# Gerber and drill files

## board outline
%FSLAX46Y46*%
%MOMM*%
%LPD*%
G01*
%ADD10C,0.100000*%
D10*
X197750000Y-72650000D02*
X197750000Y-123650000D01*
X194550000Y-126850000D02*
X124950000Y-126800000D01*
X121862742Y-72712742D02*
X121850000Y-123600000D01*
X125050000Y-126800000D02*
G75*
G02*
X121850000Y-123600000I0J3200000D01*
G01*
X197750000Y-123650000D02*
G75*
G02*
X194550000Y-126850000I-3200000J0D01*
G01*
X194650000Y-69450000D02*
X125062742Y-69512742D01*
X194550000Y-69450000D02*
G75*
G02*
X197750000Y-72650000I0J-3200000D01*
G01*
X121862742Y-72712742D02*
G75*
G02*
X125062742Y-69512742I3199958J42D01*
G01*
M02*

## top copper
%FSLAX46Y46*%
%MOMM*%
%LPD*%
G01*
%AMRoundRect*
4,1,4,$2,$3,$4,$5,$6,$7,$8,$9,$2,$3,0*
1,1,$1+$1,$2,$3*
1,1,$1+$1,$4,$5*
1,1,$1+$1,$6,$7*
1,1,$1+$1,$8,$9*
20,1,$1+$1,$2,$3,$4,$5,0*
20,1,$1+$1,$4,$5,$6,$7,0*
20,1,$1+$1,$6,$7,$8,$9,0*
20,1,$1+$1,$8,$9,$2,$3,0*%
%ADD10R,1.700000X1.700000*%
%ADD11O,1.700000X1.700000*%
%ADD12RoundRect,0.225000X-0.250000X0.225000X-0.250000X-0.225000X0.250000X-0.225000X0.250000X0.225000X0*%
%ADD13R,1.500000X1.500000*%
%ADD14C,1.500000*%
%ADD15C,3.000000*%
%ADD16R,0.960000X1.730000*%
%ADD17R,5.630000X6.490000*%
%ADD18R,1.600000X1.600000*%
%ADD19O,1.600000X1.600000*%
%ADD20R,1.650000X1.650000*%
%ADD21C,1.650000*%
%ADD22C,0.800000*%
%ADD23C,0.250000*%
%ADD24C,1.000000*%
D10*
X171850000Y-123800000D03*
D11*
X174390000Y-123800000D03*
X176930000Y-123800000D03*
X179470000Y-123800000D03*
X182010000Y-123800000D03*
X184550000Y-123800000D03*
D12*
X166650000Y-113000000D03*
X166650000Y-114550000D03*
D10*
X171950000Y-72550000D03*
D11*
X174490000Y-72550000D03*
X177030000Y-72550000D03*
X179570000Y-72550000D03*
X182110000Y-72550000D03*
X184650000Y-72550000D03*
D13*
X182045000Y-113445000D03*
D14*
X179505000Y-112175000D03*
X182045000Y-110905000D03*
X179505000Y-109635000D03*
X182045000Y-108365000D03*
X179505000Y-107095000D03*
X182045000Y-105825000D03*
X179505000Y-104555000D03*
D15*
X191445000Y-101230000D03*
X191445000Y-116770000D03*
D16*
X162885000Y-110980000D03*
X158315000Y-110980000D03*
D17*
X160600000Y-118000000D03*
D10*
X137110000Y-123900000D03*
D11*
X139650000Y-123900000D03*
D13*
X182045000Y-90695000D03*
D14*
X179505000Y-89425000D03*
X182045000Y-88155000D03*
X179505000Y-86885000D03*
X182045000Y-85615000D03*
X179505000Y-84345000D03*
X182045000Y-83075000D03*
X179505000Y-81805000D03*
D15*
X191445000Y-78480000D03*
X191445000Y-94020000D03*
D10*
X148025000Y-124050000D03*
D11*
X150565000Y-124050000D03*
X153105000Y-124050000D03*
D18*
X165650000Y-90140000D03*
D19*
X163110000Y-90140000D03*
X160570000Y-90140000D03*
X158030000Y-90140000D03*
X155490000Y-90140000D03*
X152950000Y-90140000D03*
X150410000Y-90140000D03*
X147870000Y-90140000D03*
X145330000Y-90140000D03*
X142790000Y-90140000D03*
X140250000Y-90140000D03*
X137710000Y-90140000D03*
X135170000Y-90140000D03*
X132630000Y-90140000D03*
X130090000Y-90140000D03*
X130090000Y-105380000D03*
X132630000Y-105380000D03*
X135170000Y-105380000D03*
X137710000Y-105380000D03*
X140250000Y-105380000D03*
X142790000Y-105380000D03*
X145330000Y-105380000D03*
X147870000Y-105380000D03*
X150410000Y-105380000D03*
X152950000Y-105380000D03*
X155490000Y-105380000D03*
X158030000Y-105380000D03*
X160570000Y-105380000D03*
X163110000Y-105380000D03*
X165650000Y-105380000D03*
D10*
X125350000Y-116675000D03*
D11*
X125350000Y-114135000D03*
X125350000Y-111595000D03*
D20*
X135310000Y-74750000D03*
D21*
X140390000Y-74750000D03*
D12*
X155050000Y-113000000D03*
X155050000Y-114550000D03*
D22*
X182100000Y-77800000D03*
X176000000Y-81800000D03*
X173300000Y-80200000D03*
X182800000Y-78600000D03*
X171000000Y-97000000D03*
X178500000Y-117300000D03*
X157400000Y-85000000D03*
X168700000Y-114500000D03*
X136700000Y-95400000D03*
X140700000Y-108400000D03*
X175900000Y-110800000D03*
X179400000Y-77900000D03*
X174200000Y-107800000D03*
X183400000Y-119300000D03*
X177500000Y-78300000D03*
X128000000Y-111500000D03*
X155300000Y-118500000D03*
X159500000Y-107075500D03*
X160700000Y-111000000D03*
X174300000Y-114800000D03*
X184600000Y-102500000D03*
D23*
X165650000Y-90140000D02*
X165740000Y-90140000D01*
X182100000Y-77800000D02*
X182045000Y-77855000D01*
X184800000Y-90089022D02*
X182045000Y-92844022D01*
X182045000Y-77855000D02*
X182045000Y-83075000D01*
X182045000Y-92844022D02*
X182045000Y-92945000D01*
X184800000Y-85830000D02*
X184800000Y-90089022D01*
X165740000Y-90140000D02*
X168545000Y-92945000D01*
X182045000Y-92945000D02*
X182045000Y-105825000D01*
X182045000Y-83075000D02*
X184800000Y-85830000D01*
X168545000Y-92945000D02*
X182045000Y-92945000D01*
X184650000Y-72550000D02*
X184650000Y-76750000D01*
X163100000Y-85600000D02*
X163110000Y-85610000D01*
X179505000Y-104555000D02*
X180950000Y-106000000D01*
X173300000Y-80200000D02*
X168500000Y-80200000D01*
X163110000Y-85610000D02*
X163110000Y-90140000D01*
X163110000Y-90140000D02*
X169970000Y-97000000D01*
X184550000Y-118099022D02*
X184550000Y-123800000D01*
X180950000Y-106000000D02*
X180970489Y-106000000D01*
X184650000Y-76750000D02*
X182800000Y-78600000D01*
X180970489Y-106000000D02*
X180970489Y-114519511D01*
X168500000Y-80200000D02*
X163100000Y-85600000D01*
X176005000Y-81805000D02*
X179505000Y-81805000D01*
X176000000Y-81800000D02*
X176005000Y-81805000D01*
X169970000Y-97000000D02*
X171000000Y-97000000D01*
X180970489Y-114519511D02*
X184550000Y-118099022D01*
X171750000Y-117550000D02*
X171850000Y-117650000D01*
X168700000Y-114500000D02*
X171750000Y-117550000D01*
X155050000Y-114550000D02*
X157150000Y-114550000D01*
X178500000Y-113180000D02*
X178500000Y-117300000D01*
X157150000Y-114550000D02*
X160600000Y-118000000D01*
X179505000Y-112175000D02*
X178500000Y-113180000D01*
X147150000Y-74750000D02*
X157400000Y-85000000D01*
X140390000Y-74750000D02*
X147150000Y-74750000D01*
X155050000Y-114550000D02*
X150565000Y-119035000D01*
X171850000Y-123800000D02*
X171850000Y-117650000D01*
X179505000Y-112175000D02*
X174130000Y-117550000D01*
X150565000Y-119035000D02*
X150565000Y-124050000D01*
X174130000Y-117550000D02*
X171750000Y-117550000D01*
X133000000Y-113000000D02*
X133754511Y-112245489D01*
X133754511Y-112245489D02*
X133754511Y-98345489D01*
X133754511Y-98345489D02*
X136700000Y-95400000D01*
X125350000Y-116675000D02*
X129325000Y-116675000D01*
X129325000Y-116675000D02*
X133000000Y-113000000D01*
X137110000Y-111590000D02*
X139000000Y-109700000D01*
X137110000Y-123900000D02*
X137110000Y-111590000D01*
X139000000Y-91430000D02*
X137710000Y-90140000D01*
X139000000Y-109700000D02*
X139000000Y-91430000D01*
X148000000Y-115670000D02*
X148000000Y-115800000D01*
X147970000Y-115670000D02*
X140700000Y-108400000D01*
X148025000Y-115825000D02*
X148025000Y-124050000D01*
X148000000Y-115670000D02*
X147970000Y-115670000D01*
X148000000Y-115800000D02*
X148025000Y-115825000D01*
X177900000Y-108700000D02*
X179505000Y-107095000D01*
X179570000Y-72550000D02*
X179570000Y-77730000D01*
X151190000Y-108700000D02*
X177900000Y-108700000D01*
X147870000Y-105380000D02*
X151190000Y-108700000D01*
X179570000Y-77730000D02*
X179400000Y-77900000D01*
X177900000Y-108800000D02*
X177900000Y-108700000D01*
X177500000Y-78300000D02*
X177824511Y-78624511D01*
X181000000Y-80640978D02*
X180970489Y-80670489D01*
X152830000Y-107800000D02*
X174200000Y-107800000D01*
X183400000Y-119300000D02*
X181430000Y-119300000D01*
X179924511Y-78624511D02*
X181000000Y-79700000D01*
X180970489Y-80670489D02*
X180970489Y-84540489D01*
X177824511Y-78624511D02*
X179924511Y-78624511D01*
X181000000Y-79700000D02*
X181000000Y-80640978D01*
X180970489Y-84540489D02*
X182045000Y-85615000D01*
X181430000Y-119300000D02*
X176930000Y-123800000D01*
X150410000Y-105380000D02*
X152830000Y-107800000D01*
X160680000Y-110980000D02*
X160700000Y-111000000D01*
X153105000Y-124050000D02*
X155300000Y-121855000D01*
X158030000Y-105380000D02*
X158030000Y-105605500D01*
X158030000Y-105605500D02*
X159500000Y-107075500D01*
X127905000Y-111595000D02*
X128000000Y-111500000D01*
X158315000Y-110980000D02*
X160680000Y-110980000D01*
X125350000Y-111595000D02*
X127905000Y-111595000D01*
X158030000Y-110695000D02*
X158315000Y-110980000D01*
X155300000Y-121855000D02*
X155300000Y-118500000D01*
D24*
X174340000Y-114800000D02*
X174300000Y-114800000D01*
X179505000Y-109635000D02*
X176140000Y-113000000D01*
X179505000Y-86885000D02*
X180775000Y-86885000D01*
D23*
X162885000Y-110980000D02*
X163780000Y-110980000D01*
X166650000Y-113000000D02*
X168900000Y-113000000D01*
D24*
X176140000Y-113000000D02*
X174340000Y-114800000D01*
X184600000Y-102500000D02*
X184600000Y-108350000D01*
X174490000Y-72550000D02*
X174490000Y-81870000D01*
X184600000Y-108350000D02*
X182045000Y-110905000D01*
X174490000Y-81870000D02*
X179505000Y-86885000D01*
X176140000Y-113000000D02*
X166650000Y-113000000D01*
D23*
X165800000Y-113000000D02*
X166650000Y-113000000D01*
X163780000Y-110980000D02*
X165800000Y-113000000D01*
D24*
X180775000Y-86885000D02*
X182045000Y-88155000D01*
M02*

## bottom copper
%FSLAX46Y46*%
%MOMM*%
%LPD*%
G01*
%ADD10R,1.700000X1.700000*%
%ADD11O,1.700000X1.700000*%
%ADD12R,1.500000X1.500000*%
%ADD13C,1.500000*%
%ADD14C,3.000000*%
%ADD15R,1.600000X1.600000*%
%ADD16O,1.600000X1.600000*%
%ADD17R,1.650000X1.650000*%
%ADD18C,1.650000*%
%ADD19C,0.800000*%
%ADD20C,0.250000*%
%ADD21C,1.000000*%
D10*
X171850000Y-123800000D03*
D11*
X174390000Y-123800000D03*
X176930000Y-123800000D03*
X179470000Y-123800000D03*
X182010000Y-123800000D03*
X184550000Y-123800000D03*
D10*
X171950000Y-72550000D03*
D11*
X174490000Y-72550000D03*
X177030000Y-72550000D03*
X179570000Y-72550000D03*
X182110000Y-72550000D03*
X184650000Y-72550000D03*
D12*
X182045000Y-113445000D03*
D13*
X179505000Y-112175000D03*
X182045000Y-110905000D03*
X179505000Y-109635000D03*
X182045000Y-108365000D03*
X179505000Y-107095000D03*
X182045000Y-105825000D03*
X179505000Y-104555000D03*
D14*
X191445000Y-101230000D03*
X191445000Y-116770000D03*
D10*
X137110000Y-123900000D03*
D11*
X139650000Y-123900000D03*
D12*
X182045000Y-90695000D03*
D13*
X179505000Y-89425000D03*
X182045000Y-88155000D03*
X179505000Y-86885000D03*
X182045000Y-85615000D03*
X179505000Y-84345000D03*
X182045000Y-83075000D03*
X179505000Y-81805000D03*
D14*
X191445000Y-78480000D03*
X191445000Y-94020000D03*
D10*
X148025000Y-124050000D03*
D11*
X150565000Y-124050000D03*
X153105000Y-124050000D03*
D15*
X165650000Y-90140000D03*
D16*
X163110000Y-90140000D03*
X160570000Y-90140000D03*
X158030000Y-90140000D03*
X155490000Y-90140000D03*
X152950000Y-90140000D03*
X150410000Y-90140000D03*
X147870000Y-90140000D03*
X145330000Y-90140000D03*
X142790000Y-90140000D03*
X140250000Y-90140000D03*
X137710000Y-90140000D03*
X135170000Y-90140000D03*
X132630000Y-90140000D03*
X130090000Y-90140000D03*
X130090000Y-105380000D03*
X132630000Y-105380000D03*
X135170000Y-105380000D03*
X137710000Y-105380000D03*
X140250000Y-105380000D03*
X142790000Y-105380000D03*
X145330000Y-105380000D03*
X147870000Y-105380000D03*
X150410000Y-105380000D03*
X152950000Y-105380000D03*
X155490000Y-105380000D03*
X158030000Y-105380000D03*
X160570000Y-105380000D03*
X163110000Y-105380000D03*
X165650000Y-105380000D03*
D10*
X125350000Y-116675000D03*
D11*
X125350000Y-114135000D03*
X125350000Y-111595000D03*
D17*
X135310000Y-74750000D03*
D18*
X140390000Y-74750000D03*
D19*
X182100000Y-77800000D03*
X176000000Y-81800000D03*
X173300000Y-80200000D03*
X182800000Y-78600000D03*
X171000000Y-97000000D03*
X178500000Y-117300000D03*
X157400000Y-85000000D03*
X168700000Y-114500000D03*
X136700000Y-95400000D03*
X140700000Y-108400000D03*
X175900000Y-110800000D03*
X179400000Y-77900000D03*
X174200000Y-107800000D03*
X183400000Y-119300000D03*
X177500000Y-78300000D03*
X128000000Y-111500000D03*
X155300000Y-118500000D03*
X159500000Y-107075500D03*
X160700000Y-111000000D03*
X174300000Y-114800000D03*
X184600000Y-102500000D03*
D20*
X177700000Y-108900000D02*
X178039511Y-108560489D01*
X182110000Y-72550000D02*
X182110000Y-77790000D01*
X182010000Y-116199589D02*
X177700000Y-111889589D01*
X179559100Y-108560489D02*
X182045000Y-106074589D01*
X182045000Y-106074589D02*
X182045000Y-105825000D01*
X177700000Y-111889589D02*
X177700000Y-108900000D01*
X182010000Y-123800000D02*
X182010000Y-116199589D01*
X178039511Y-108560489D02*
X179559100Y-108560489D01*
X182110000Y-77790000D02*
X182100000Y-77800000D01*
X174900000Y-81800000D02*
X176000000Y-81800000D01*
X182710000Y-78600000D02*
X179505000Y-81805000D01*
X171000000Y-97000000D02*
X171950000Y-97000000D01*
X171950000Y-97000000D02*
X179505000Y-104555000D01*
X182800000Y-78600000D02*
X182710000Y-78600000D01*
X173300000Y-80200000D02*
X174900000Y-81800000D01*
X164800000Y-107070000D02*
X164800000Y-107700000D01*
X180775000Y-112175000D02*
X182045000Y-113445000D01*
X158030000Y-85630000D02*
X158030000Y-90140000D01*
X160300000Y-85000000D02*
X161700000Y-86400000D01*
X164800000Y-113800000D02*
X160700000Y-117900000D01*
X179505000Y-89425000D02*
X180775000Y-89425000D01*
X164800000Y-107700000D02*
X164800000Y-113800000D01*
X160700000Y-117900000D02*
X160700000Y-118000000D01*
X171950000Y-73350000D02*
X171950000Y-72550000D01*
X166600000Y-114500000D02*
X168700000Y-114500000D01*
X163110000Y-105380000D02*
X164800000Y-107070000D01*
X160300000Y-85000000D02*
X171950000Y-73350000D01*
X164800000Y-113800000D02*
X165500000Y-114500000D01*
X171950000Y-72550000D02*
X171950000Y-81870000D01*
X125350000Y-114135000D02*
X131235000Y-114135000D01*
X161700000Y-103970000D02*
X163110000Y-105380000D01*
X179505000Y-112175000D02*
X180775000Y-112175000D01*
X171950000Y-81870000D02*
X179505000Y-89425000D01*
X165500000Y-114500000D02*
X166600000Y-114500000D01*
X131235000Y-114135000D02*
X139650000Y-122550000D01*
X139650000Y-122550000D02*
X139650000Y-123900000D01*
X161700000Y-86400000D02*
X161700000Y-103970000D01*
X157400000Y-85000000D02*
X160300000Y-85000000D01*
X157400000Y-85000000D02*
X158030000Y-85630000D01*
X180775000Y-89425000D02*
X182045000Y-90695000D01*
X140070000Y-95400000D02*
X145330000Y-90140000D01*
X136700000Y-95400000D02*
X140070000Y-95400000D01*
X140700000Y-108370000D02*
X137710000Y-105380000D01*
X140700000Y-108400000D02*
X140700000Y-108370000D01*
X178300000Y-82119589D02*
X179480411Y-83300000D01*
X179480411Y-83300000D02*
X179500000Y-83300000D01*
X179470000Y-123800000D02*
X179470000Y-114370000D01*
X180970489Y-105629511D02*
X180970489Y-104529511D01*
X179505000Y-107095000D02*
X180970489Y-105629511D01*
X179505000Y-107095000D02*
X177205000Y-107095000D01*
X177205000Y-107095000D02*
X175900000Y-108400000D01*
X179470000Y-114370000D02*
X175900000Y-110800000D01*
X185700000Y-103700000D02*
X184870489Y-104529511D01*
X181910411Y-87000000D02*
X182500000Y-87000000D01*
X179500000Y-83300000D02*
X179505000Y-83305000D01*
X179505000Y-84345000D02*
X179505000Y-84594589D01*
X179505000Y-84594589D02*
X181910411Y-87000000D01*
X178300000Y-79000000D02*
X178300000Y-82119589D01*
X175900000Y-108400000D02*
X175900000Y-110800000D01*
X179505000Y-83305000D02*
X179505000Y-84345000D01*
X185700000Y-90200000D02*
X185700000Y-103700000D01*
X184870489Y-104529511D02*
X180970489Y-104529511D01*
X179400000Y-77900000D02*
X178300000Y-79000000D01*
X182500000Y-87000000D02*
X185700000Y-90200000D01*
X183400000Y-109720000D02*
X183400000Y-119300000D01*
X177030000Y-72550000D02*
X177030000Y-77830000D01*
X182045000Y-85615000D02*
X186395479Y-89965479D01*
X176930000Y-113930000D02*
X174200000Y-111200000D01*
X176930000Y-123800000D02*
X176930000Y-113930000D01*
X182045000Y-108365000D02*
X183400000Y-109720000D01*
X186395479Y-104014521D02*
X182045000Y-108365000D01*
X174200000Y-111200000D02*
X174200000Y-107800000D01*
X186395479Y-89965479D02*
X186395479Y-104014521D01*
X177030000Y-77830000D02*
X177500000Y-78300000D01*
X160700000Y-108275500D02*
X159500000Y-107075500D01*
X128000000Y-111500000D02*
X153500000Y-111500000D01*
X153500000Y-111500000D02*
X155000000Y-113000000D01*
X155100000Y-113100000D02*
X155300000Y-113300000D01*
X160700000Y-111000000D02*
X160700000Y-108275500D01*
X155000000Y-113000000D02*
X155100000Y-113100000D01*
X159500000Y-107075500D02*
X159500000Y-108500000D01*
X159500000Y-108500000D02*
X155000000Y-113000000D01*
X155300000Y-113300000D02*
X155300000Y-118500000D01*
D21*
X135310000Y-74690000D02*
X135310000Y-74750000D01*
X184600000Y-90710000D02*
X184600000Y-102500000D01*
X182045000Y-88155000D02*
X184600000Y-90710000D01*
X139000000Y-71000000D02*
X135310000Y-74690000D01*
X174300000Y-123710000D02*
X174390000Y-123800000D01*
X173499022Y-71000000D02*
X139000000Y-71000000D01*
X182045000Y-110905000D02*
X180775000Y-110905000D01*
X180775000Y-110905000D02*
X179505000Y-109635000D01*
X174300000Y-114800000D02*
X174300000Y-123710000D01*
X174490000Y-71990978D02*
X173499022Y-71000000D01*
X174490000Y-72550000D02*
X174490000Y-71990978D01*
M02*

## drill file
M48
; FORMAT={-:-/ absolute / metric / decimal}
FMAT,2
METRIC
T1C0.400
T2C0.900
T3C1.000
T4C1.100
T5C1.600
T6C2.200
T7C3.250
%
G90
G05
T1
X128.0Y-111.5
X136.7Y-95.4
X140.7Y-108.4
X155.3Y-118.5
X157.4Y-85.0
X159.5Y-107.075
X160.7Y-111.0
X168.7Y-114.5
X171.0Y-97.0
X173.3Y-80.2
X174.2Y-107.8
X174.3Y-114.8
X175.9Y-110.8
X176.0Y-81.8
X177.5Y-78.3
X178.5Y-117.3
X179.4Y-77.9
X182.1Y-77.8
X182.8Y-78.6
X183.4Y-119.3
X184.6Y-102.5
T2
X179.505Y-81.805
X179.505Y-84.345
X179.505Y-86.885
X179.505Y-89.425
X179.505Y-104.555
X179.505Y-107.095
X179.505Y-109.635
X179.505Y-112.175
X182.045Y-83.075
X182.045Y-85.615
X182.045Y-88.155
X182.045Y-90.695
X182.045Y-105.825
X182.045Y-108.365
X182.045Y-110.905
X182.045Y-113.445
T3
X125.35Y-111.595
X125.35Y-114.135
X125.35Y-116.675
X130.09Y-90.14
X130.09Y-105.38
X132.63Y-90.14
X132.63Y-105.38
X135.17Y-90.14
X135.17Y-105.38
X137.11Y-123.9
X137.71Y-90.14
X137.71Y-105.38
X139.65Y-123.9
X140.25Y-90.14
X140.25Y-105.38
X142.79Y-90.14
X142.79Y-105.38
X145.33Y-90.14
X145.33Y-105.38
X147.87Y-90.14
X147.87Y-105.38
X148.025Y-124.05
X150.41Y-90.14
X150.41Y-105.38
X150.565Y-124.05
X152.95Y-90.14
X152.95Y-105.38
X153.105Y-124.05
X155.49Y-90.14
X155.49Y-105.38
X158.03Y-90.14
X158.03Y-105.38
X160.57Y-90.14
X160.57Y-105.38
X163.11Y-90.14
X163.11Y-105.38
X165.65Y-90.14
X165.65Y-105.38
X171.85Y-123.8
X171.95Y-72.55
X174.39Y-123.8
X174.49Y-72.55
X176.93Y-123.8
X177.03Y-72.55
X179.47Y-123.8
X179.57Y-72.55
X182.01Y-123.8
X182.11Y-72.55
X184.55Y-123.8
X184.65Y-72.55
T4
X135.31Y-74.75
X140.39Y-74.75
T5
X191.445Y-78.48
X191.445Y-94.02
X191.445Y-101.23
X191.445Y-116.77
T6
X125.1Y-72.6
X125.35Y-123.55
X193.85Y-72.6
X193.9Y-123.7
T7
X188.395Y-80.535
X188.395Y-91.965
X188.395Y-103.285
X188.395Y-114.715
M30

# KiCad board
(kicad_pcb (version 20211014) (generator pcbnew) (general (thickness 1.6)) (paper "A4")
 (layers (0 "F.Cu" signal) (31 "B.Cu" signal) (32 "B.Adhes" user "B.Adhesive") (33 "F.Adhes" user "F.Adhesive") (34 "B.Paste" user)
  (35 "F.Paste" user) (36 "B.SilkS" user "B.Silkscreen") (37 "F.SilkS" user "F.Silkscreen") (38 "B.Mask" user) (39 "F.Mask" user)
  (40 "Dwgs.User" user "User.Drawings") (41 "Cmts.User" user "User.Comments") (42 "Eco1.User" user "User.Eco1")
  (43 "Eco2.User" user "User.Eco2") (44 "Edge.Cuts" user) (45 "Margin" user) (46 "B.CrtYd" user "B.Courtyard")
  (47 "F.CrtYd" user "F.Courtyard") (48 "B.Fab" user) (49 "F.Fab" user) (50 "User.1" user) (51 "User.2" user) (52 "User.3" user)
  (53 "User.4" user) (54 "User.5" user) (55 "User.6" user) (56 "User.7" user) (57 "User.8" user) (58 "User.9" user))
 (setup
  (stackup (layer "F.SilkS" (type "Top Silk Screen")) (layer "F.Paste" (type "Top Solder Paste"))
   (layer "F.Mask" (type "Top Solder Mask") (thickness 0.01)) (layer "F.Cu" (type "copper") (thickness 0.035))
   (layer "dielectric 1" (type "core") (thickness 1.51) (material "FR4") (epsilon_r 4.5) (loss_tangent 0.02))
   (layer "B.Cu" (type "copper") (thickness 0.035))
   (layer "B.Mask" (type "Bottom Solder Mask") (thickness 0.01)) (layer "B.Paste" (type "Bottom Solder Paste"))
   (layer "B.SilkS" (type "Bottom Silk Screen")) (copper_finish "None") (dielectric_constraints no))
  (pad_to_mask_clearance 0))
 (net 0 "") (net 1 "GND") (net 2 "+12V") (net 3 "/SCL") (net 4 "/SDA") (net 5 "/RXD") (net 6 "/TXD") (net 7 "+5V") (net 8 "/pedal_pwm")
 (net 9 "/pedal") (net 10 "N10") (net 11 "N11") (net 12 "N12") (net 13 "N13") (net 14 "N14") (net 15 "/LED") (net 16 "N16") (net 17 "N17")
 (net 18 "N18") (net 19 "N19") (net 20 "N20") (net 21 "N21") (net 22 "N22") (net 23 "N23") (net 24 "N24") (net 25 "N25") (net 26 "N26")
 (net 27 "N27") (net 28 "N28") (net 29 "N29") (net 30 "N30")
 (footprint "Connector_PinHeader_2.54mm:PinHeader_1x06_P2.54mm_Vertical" (layer "F.Cu") (at 171.85 123.8 90)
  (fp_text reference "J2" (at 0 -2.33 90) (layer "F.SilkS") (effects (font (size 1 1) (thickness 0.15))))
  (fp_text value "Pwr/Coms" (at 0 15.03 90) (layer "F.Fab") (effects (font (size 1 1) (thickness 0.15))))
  (pad "1" thru_hole rect (at 0 0 90) (size 1.7 1.7) (drill 1) (layers *.Cu *.Mask) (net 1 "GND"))
  (pad "2" thru_hole oval (at 0 2.54 90) (size 1.7 1.7) (drill 1) (layers *.Cu *.Mask) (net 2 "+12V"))
  (pad "3" thru_hole oval (at 0 5.08 90) (size 1.7 1.7) (drill 1) (layers *.Cu *.Mask) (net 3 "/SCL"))
  (pad "4" thru_hole oval (at 0 7.62 90) (size 1.7 1.7) (drill 1) (layers *.Cu *.Mask) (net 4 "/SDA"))
  (pad "5" thru_hole oval (at 0 10.16 90) (size 1.7 1.7) (drill 1) (layers *.Cu *.Mask) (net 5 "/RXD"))
  (pad "6" thru_hole oval (at 0 12.7 90) (size 1.7 1.7) (drill 1) (layers *.Cu *.Mask) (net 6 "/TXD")))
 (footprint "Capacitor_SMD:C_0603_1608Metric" (layer "F.Cu") (at 166.65 113.775 -90)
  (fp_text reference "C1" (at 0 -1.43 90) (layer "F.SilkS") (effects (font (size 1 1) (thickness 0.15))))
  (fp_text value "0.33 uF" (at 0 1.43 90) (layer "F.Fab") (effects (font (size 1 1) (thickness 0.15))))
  (pad "1" smd roundrect (at -0.775 0 270) (size 0.9 0.95) (layers "F.Cu" "F.Paste" "F.Mask") (roundrect_rratio 0.25) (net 2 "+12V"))
  (pad "2" smd roundrect (at 0.775 0 270) (size 0.9 0.95) (layers "F.Cu" "F.Paste" "F.Mask") (roundrect_rratio 0.25) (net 1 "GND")))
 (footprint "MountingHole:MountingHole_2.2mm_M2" (layer "F.Cu") (at 193.9 123.7)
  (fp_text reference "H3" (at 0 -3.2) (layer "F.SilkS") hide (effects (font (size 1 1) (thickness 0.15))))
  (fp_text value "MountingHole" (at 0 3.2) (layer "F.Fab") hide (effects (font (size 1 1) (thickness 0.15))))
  (pad "" np_thru_hole circle (at 0 0) (size 2.2 2.2) (drill 2.2) (layers *.Cu *.Mask)))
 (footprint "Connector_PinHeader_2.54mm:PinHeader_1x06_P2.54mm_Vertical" (layer "F.Cu") (at 171.95 72.55 90)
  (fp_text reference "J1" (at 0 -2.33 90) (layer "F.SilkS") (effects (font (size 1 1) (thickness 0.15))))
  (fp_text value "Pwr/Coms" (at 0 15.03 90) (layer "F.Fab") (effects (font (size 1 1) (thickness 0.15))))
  (pad "1" thru_hole rect (at 0 0 90) (size 1.7 1.7) (drill 1) (layers *.Cu *.Mask) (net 1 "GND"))
  (pad "2" thru_hole oval (at 0 2.54 90) (size 1.7 1.7) (drill 1) (layers *.Cu *.Mask) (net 2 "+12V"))
  (pad "3" thru_hole oval (at 0 5.08 90) (size 1.7 1.7) (drill 1) (layers *.Cu *.Mask) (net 3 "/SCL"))
  (pad "4" thru_hole oval (at 0 7.62 90) (size 1.7 1.7) (drill 1) (layers *.Cu *.Mask) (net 4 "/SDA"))
  (pad "5" thru_hole oval (at 0 10.16 90) (size 1.7 1.7) (drill 1) (layers *.Cu *.Mask) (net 5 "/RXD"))
  (pad "6" thru_hole oval (at 0 12.7 90) (size 1.7 1.7) (drill 1) (layers *.Cu *.Mask) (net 6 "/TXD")))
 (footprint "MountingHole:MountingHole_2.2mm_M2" (layer "F.Cu") (at 125.1 72.6)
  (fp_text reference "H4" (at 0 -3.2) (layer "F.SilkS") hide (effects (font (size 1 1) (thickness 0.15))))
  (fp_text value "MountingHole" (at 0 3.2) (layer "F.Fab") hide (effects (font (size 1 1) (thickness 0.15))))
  (pad "" np_thru_hole circle (at 0 0) (size 2.2 2.2) (drill 2.2) (layers *.Cu *.Mask)))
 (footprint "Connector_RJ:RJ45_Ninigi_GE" (layer "F.Cu") (at 182.045 113.445 90)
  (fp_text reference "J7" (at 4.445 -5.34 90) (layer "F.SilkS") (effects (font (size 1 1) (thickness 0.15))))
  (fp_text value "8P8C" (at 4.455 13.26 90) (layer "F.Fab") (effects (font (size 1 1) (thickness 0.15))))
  (pad "" np_thru_hole circle (at 10.16 6.35 270) (size 3.25 3.25) (drill 3.25) (layers *.Cu *.Mask))
  (pad "" np_thru_hole circle (at -1.27 6.35 90) (size 3.25 3.25) (drill 3.25) (layers *.Cu *.Mask))
  (pad "1" thru_hole rect (at 0 0 270) (size 1.5 1.5) (drill 0.9) (layers *.Cu *.Mask) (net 1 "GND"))
  (pad "2" thru_hole circle (at 1.27 -2.54 270) (size 1.5 1.5) (drill 0.9) (layers *.Cu *.Mask) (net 1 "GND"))
  (pad "3" thru_hole circle (at 2.54 0 270) (size 1.5 1.5) (drill 0.9) (layers *.Cu *.Mask) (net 2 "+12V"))
  (pad "4" thru_hole circle (at 3.81 -2.54 270) (size 1.5 1.5) (drill 0.9) (layers *.Cu *.Mask) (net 2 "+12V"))
  (pad "5" thru_hole circle (at 5.08 0 270) (size 1.5 1.5) (drill 0.9) (layers *.Cu *.Mask) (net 3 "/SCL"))
  (pad "6" thru_hole circle (at 6.35 -2.54 270) (size 1.5 1.5) (drill 0.9) (layers *.Cu *.Mask) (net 4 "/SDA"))
  (pad "7" thru_hole circle (at 7.62 0 270) (size 1.5 1.5) (drill 0.9) (layers *.Cu *.Mask) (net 5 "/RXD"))
  (pad "8" thru_hole circle (at 8.89 -2.54 270) (size 1.5 1.5) (drill 0.9) (layers *.Cu *.Mask) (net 6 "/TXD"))
  (pad "SH" thru_hole circle (at 12.215 9.4 270) (size 3 3) (drill 1.6) (layers *.Cu *.Mask))
  (pad "SH" thru_hole circle (at -3.325 9.4 90) (size 3 3) (drill 1.6) (layers *.Cu *.Mask)))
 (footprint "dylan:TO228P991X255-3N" (layer "F.Cu") (at 160.6 115.68 -90)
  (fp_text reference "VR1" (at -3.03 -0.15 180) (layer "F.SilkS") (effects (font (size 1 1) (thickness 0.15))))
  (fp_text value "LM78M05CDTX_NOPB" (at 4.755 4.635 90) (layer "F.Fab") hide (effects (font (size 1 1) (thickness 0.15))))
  (pad "1" smd rect locked (at -4.7 -2.285 270) (size 1.73 0.96) (layers "F.Cu" "F.Paste" "F.Mask") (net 2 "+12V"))
  (pad "3" smd rect locked (at -4.7 2.285 270) (size 1.73 0.96) (layers "F.Cu" "F.Paste" "F.Mask") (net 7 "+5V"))
  (pad "4" smd rect locked (at 2.32 0 270) (size 6.49 5.63) (layers "F.Cu" "F.Mask") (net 1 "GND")))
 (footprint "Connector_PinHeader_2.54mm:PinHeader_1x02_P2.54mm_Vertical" (layer "F.Cu") (at 137.11 123.9 90)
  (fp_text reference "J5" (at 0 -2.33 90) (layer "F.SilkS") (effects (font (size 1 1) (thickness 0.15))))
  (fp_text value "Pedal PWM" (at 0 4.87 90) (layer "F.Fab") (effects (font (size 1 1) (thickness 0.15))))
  (pad "1" thru_hole rect (at 0 0 90) (size 1.7 1.7) (drill 1) (layers *.Cu *.Mask) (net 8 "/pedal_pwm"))
  (pad "2" thru_hole oval (at 0 2.54 90) (size 1.7 1.7) (drill 1) (layers *.Cu *.Mask) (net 1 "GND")))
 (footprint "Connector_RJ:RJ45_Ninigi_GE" (layer "F.Cu") (at 182.045 90.695 90)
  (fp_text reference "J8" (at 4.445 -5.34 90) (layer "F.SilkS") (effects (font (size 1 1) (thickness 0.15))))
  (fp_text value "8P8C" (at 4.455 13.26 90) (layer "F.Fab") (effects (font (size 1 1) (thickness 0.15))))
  (pad "" np_thru_hole circle (at 10.16 6.35 270) (size 3.25 3.25) (drill 3.25) (layers *.Cu *.Mask))
  (pad "" np_thru_hole circle (at -1.27 6.35 90) (size 3.25 3.25) (drill 3.25) (layers *.Cu *.Mask))
  (pad "1" thru_hole rect (at 0 0 270) (size 1.5 1.5) (drill 0.9) (layers *.Cu *.Mask) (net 1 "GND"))
  (pad "2" thru_hole circle (at 1.27 -2.54 270) (size 1.5 1.5) (drill 0.9) (layers *.Cu *.Mask) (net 1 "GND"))
  (pad "3" thru_hole circle (at 2.54 0 270) (size 1.5 1.5) (drill 0.9) (layers *.Cu *.Mask) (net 2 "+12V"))
  (pad "4" thru_hole circle (at 3.81 -2.54 270) (size 1.5 1.5) (drill 0.9) (layers *.Cu *.Mask) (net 2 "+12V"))
  (pad "5" thru_hole circle (at 5.08 0 270) (size 1.5 1.5) (drill 0.9) (layers *.Cu *.Mask) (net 3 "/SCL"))
  (pad "6" thru_hole circle (at 6.35 -2.54 270) (size 1.5 1.5) (drill 0.9) (layers *.Cu *.Mask) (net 4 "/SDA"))
  (pad "7" thru_hole circle (at 7.62 0 270) (size 1.5 1.5) (drill 0.9) (layers *.Cu *.Mask) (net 5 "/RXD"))
  (pad "8" thru_hole circle (at 8.89 -2.54 270) (size 1.5 1.5) (drill 0.9) (layers *.Cu *.Mask) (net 6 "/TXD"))
  (pad "SH" thru_hole circle (at 12.215 9.4 270) (size 3 3) (drill 1.6) (layers *.Cu *.Mask))
  (pad "SH" thru_hole circle (at -3.325 9.4 90) (size 3 3) (drill 1.6) (layers *.Cu *.Mask)))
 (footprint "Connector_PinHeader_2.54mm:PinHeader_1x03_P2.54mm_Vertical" (layer "F.Cu") (at 148.025 124.05 90)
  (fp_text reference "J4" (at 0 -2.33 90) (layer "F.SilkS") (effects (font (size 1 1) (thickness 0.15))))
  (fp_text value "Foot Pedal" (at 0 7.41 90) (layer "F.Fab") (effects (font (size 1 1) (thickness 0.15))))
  (pad "1" thru_hole rect (at 0 0 90) (size 1.7 1.7) (drill 1) (layers *.Cu *.Mask) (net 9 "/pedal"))
  (pad "2" thru_hole oval (at 0 2.54 90) (size 1.7 1.7) (drill 1) (layers *.Cu *.Mask) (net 1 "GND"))
  (pad "3" thru_hole oval (at 0 5.08 90) (size 1.7 1.7) (drill 1) (layers *.Cu *.Mask) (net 7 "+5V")))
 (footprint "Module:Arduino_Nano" (layer "F.Cu") (at 165.65 90.14 -90)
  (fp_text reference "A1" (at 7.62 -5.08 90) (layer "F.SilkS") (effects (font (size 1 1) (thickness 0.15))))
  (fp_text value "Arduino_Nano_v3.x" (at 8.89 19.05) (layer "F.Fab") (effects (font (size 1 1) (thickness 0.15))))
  (pad "1" thru_hole rect (at 0 0 270) (size 1.6 1.6) (drill 1) (layers *.Cu *.Mask) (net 5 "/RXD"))
  (pad "2" thru_hole oval (at 0 2.54 270) (size 1.6 1.6) (drill 1) (layers *.Cu *.Mask) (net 6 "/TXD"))
  (pad "3" thru_hole oval (at 0 5.08 270) (size 1.6 1.6) (drill 1) (layers *.Cu *.Mask) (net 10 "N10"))
  (pad "4" thru_hole oval (at 0 7.62 270) (size 1.6 1.6) (drill 1) (layers *.Cu *.Mask) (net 1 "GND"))
  (pad "5" thru_hole oval (at 0 10.16 270) (size 1.6 1.6) (drill 1) (layers *.Cu *.Mask) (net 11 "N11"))
  (pad "6" thru_hole oval (at 0 12.7 270) (size 1.6 1.6) (drill 1) (layers *.Cu *.Mask) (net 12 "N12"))
  (pad "7" thru_hole oval (at 0 15.24 270) (size 1.6 1.6) (drill 1) (layers *.Cu *.Mask) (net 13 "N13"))
  (pad "8" thru_hole oval (at 0 17.78 270) (size 1.6 1.6) (drill 1) (layers *.Cu *.Mask) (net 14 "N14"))
  (pad "9" thru_hole oval (at 0 20.32 270) (size 1.6 1.6) (drill 1) (layers *.Cu *.Mask) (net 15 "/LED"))
  (pad "10" thru_hole oval (at 0 22.86 270) (size 1.6 1.6) (drill 1) (layers *.Cu *.Mask) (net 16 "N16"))
  (pad "11" thru_hole oval (at 0 25.4 270) (size 1.6 1.6) (drill 1) (layers *.Cu *.Mask) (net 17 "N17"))
  (pad "12" thru_hole oval (at 0 27.94 270) (size 1.6 1.6) (drill 1) (layers *.Cu *.Mask) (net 8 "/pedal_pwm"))
  (pad "13" thru_hole oval (at 0 30.48 270) (size 1.6 1.6) (drill 1) (layers *.Cu *.Mask) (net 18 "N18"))
  (pad "14" thru_hole oval (at 0 33.02 270) (size 1.6 1.6) (drill 1) (layers *.Cu *.Mask) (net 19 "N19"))
  (pad "15" thru_hole oval (at 0 35.56 270) (size 1.6 1.6) (drill 1) (layers *.Cu *.Mask) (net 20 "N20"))
  (pad "16" thru_hole oval (at 15.24 35.56 270) (size 1.6 1.6) (drill 1) (layers *.Cu *.Mask) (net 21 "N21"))
  (pad "17" thru_hole oval (at 15.24 33.02 270) (size 1.6 1.6) (drill 1) (layers *.Cu *.Mask) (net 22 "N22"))
  (pad "18" thru_hole oval (at 15.24 30.48 270) (size 1.6 1.6) (drill 1) (layers *.Cu *.Mask) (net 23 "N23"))
  (pad "19" thru_hole oval (at 15.24 27.94 270) (size 1.6 1.6) (drill 1) (layers *.Cu *.Mask) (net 9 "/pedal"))
  (pad "20" thru_hole oval (at 15.24 25.4 270) (size 1.6 1.6) (drill 1) (layers *.Cu *.Mask) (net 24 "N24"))
  (pad "21" thru_hole oval (at 15.24 22.86 270) (size 1.6 1.6) (drill 1) (layers *.Cu *.Mask) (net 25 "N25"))
  (pad "22" thru_hole oval (at 15.24 20.32 270) (size 1.6 1.6) (drill 1) (layers *.Cu *.Mask) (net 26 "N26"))
  (pad "23" thru_hole oval (at 15.24 17.78 270) (size 1.6 1.6) (drill 1) (layers *.Cu *.Mask) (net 4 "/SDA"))
  (pad "24" thru_hole oval (at 15.24 15.24 270) (size 1.6 1.6) (drill 1) (layers *.Cu *.Mask) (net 3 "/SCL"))
  (pad "25" thru_hole oval (at 15.24 12.7 270) (size 1.6 1.6) (drill 1) (layers *.Cu *.Mask) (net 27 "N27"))
  (pad "26" thru_hole oval (at 15.24 10.16 270) (size 1.6 1.6) (drill 1) (layers *.Cu *.Mask) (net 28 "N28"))
  (pad "27" thru_hole oval (at 15.24 7.62 270) (size 1.6 1.6) (drill 1) (layers *.Cu *.Mask) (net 7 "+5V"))
  (pad "28" thru_hole oval (at 15.24 5.08 270) (size 1.6 1.6) (drill 1) (layers *.Cu *.Mask) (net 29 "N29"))
  (pad "29" thru_hole oval (at 15.24 2.54 270) (size 1.6 1.6) (drill 1) (layers *.Cu *.Mask) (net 1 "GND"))
  (pad "30" thru_hole oval (at 15.24 0 270) (size 1.6 1.6) (drill 1) (layers *.Cu *.Mask) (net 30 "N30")))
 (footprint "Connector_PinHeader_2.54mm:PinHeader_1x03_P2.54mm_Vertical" (layer "F.Cu") (at 125.35 116.675 180)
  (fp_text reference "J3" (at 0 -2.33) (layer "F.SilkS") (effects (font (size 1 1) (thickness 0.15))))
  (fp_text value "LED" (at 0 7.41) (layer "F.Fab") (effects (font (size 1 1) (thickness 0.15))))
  (pad "1" thru_hole rect (at 0 0 180) (size 1.7 1.7) (drill 1) (layers *.Cu *.Mask) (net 15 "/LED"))
  (pad "2" thru_hole oval (at 0 2.54 180) (size 1.7 1.7) (drill 1) (layers *.Cu *.Mask) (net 1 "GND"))
  (pad "3" thru_hole oval (at 0 5.08 180) (size 1.7 1.7) (drill 1) (layers *.Cu *.Mask) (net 7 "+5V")))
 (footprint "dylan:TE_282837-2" (layer "F.Cu") (at 137.85 74.75)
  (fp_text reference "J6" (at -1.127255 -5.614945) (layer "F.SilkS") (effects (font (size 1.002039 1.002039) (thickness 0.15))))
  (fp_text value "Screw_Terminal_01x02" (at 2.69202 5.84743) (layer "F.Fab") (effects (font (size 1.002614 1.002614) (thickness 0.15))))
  (pad "1" thru_hole rect locked (at -2.54 0) (size 1.65 1.65) (drill 1.1) (layers *.Cu *.Mask) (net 2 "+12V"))
  (pad "2" thru_hole circle locked (at 2.54 0) (size 1.65 1.65) (drill 1.1) (layers *.Cu *.Mask) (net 1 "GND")))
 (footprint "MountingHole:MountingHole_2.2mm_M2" (layer "F.Cu") (at 193.85 72.6)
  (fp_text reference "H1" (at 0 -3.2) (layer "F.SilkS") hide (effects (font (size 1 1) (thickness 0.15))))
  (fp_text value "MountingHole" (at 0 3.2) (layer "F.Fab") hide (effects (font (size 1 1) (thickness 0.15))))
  (pad "" np_thru_hole circle (at 0 0) (size 2.2 2.2) (drill 2.2) (layers *.Cu *.Mask)))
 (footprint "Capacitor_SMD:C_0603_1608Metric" (layer "F.Cu") (at 155.05 113.775 -90)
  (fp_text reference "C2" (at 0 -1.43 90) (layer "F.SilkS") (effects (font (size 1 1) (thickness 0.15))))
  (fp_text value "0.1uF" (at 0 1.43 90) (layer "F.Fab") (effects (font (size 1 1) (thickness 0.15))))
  (pad "1" smd roundrect (at -0.775 0 270) (size 0.9 0.95) (layers "F.Cu" "F.Paste" "F.Mask") (roundrect_rratio 0.25) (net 7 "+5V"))
  (pad "2" smd roundrect (at 0.775 0 270) (size 0.9 0.95) (layers "F.Cu" "F.Paste" "F.Mask") (roundrect_rratio 0.25) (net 1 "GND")))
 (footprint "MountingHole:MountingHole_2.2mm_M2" (layer "F.Cu") (at 125.35 123.55)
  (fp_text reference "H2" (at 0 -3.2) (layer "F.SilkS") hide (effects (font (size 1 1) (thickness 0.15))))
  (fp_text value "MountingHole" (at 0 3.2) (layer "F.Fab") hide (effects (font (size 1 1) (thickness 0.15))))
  (pad "" np_thru_hole circle (at 0 0) (size 2.2 2.2) (drill 2.2) (layers *.Cu *.Mask)))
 (gr_line (start 197.75 72.65) (end 197.75 123.65) (layer "Edge.Cuts") (width 0.1))
 (gr_line (start 194.55 126.85) (end 124.95 126.8) (layer "Edge.Cuts") (width 0.1))
 (gr_line (start 121.862742 72.712742) (end 121.85 123.6) (layer "Edge.Cuts") (width 0.1))
 (gr_arc (start 125.05 126.8) (mid 122.787258 125.862742) (end 121.85 123.6) (layer "Edge.Cuts") (width 0.1))
 (gr_arc (start 197.75 123.65) (mid 196.812742 125.912742) (end 194.55 126.85) (layer "Edge.Cuts") (width 0.1))
 (gr_line (start 194.65 69.45) (end 125.062742 69.512742) (layer "Edge.Cuts") (width 0.1))
 (gr_arc (start 194.55 69.45) (mid 196.812742 70.387258) (end 197.75 72.65) (layer "Edge.Cuts") (width 0.1))
 (gr_arc (start 121.862742 72.712742) (mid 122.8 70.45) (end 125.062742 69.512742) (layer "Edge.Cuts") (width 0.1))
 (segment (start 165.65 90.14) (end 165.74 90.14) (width 0.25) (layer "F.Cu") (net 5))
 (segment (start 182.1 77.8) (end 182.045 77.855) (width 0.25) (layer "F.Cu") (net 5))
 (segment (start 184.8 90.089022) (end 182.045 92.844022) (width 0.25) (layer "F.Cu") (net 5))
 (segment (start 182.045 77.855) (end 182.045 83.075) (width 0.25) (layer "F.Cu") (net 5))
 (segment (start 182.045 92.844022) (end 182.045 92.945) (width 0.25) (layer "F.Cu") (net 5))
 (segment (start 184.8 85.83) (end 184.8 90.089022) (width 0.25) (layer "F.Cu") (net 5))
 (segment (start 165.74 90.14) (end 168.545 92.945) (width 0.25) (layer "F.Cu") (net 5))
 (segment (start 182.045 92.945) (end 182.045 105.825) (width 0.25) (layer "F.Cu") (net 5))
 (segment (start 182.045 83.075) (end 184.8 85.83) (width 0.25) (layer "F.Cu") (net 5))
 (segment (start 168.545 92.945) (end 182.045 92.945) (width 0.25) (layer "F.Cu") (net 5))
 (via (at 182.1 77.8) (size 0.8) (drill 0.4) (layers "F.Cu" "B.Cu") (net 5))
 (segment (start 177.7 108.9) (end 178.039511 108.560489) (width 0.25) (layer "B.Cu") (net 5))
 (segment (start 182.11 72.55) (end 182.11 77.79) (width 0.25) (layer "B.Cu") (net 5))
 (segment (start 182.01 116.199589) (end 177.7 111.889589) (width 0.25) (layer "B.Cu") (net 5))
 (segment (start 179.5591 108.560489) (end 182.045 106.074589) (width 0.25) (layer "B.Cu") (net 5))
 (segment (start 182.045 106.074589) (end 182.045 105.825) (width 0.25) (layer "B.Cu") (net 5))
 (segment (start 177.7 111.889589) (end 177.7 108.9) (width 0.25) (layer "B.Cu") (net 5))
 (segment (start 182.01 123.8) (end 182.01 116.199589) (width 0.25) (layer "B.Cu") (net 5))
 (segment (start 178.039511 108.560489) (end 179.5591 108.560489) (width 0.25) (layer "B.Cu") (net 5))
 (segment (start 182.11 77.79) (end 182.1 77.8) (width 0.25) (layer "B.Cu") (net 5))
 (segment (start 184.65 72.55) (end 184.65 76.75) (width 0.25) (layer "F.Cu") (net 6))
 (segment (start 163.1 85.6) (end 163.11 85.61) (width 0.25) (layer "F.Cu") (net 6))
 (segment (start 179.505 104.555) (end 180.95 106) (width 0.25) (layer "F.Cu") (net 6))
 (segment (start 173.3 80.2) (end 168.5 80.2) (width 0.25) (layer "F.Cu") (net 6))
 (segment (start 163.11 85.61) (end 163.11 90.14) (width 0.25) (layer "F.Cu") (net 6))
 (segment (start 163.11 90.14) (end 169.97 97) (width 0.25) (layer "F.Cu") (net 6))
 (segment (start 184.55 118.099022) (end 184.55 123.8) (width 0.25) (layer "F.Cu") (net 6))
 (segment (start 180.95 106) (end 180.970489 106) (width 0.25) (layer "F.Cu") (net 6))
 (segment (start 184.65 76.75) (end 182.8 78.6) (width 0.25) (layer "F.Cu") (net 6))
 (segment (start 180.970489 106) (end 180.970489 114.519511) (width 0.25) (layer "F.Cu") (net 6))
 (segment (start 168.5 80.2) (end 163.1 85.6) (width 0.25) (layer "F.Cu") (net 6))
 (segment (start 176.005 81.805) (end 179.505 81.805) (width 0.25) (layer "F.Cu") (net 6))
 (segment (start 176 81.8) (end 176.005 81.805) (width 0.25) (layer "F.Cu") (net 6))
 (segment (start 169.97 97) (end 171 97) (width 0.25) (layer "F.Cu") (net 6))
 (segment (start 180.970489 114.519511) (end 184.55 118.099022) (width 0.25) (layer "F.Cu") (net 6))
 (via (at 176 81.8) (size 0.8) (drill 0.4) (layers "F.Cu" "B.Cu") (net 6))
 (via (at 173.3 80.2) (size 0.8) (drill 0.4) (layers "F.Cu" "B.Cu") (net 6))
 (via (at 182.8 78.6) (size 0.8) (drill 0.4) (layers "F.Cu" "B.Cu") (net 6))
 (via (at 171 97) (size 0.8) (drill 0.4) (layers "F.Cu" "B.Cu") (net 6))
 (segment (start 174.9 81.8) (end 176 81.8) (width 0.25) (layer "B.Cu") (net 6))
 (segment (start 182.71 78.6) (end 179.505 81.805) (width 0.25) (layer "B.Cu") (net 6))
 (segment (start 171 97) (end 171.95 97) (width 0.25) (layer "B.Cu") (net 6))
 (segment (start 171.95 97) (end 179.505 104.555) (width 0.25) (layer "B.Cu") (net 6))
 (segment (start 182.8 78.6) (end 182.71 78.6) (width 0.25) (layer "B.Cu") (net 6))
 (segment (start 173.3 80.2) (end 174.9 81.8) (width 0.25) (layer "B.Cu") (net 6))
 (segment (start 171.75 117.55) (end 171.85 117.65) (width 0.25) (layer "F.Cu") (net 1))
 (segment (start 168.7 114.5) (end 171.75 117.55) (width 0.25) (layer "F.Cu") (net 1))
 (segment (start 155.05 114.55) (end 157.15 114.55) (width 0.25) (layer "F.Cu") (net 1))
 (segment (start 178.5 113.18) (end 178.5 117.3) (width 0.25) (layer "F.Cu") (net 1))
 (segment (start 157.15 114.55) (end 160.6 118) (width 0.25) (layer "F.Cu") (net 1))
 (segment (start 179.505 112.175) (end 178.5 113.18) (width 0.25) (layer "F.Cu") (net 1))
 (segment (start 147.15 74.75) (end 157.4 85) (width 0.25) (layer "F.Cu") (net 1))
 (segment (start 140.39 74.75) (end 147.15 74.75) (width 0.25) (layer "F.Cu") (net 1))
 (segment (start 155.05 114.55) (end 150.565 119.035) (width 0.25) (layer "F.Cu") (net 1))
 (segment (start 171.85 123.8) (end 171.85 117.65) (width 0.25) (layer "F.Cu") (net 1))
 (segment (start 179.505 112.175) (end 174.13 117.55) (width 0.25) (layer "F.Cu") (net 1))
 (segment (start 150.565 119.035) (end 150.565 124.05) (width 0.25) (layer "F.Cu") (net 1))
 (segment (start 174.13 117.55) (end 171.75 117.55) (width 0.25) (layer "F.Cu") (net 1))
 (via (at 178.5 117.3) (size 0.8) (drill 0.4) (layers "F.Cu" "B.Cu") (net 1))
 (via (at 157.4 85) (size 0.8) (drill 0.4) (layers "F.Cu" "B.Cu") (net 1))
 (via (at 168.7 114.5) (size 0.8) (drill 0.4) (layers "F.Cu" "B.Cu") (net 1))
 (segment (start 164.8 107.07) (end 164.8 107.7) (width 0.25) (layer "B.Cu") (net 1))
 (segment (start 180.775 112.175) (end 182.045 113.445) (width 0.25) (layer "B.Cu") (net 1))
 (segment (start 158.03 85.63) (end 158.03 90.14) (width 0.25) (layer "B.Cu") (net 1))
 (segment (start 160.3 85) (end 161.7 86.4) (width 0.25) (layer "B.Cu") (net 1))
 (segment (start 164.8 113.8) (end 160.7 117.9) (width 0.25) (layer "B.Cu") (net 1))
 (segment (start 179.505 89.425) (end 180.775 89.425) (width 0.25) (layer "B.Cu") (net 1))
 (segment (start 164.8 107.7) (end 164.8 113.8) (width 0.25) (layer "B.Cu") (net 1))
 (segment (start 160.7 117.9) (end 160.7 118) (width 0.25) (layer "B.Cu") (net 1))
 (segment (start 171.95 73.35) (end 171.95 72.55) (width 0.25) (layer "B.Cu") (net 1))
 (segment (start 166.6 114.5) (end 168.7 114.5) (width 0.25) (layer "B.Cu") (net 1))
 (segment (start 163.11 105.38) (end 164.8 107.07) (width 0.25) (layer "B.Cu") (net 1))
 (segment (start 160.3 85) (end 171.95 73.35) (width 0.25) (layer "B.Cu") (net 1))
 (segment (start 164.8 113.8) (end 165.5 114.5) (width 0.25) (layer "B.Cu") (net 1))
 (segment (start 171.95 72.55) (end 171.95 81.87) (width 0.25) (layer "B.Cu") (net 1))
 (segment (start 125.35 114.135) (end 131.235 114.135) (width 0.25) (layer "B.Cu") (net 1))
 (segment (start 161.7 103.97) (end 163.11 105.38) (width 0.25) (layer "B.Cu") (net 1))
 (segment (start 179.505 112.175) (end 180.775 112.175) (width 0.25) (layer "B.Cu") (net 1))
 (segment (start 171.95 81.87) (end 179.505 89.425) (width 0.25) (layer "B.Cu") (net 1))
 (segment (start 165.5 114.5) (end 166.6 114.5) (width 0.25) (layer "B.Cu") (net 1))
 (segment (start 131.235 114.135) (end 139.65 122.55) (width 0.25) (layer "B.Cu") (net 1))
 (segment (start 139.65 122.55) (end 139.65 123.9) (width 0.25) (layer "B.Cu") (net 1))
 (segment (start 161.7 86.4) (end 161.7 103.97) (width 0.25) (layer "B.Cu") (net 1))
 (segment (start 157.4 85) (end 160.3 85) (width 0.25) (layer "B.Cu") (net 1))
 (segment (start 157.4 85) (end 158.03 85.63) (width 0.25) (layer "B.Cu") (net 1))
 (segment (start 180.775 89.425) (end 182.045 90.695) (width 0.25) (layer "B.Cu") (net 1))
 (segment (start 133 113) (end 133.754511 112.245489) (width 0.25) (layer "F.Cu") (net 15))
 (segment (start 133.754511 112.245489) (end 133.754511 98.345489) (width 0.25) (layer "F.Cu") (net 15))
 (segment (start 133.754511 98.345489) (end 136.7 95.4) (width 0.25) (layer "F.Cu") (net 15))
 (segment (start 125.35 116.675) (end 129.325 116.675) (width 0.25) (layer "F.Cu") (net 15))
 (segment (start 129.325 116.675) (end 133 113) (width 0.25) (layer "F.Cu") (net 15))
 (via (at 136.7 95.4) (size 0.8) (drill 0.4) (layers "F.Cu" "B.Cu") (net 15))
 (segment (start 140.07 95.4) (end 145.33 90.14) (width 0.25) (layer "B.Cu") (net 15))
 (segment (start 136.7 95.4) (end 140.07 95.4) (width 0.25) (layer "B.Cu") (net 15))
 (segment (start 137.11 111.59) (end 139 109.7) (width 0.25) (layer "F.Cu") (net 8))
 (segment (start 137.11 123.9) (end 137.11 111.59) (width 0.25) (layer "F.Cu") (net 8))
 (segment (start 139 91.43) (end 137.71 90.14) (width 0.25) (layer "F.Cu") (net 8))
 (segment (start 139 109.7) (end 139 91.43) (width 0.25) (layer "F.Cu") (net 8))
 (segment (start 148 115.67) (end 148 115.8) (width 0.25) (layer "F.Cu") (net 9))
 (segment (start 147.97 115.67) (end 140.7 108.4) (width 0.25) (layer "F.Cu") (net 9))
 (segment (start 148.025 115.825) (end 148.025 124.05) (width 0.25) (layer "F.Cu") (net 9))
 (segment (start 148 115.67) (end 147.97 115.67) (width 0.25) (layer "F.Cu") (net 9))
 (segment (start 148 115.8) (end 148.025 115.825) (width 0.25) (layer "F.Cu") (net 9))
 (via (at 140.7 108.4) (size 0.8) (drill 0.4) (layers "F.Cu" "B.Cu") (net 9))
 (segment (start 140.7 108.37) (end 137.71 105.38) (width 0.25) (layer "B.Cu") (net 9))
 (segment (start 140.7 108.4) (end 140.7 108.37) (width 0.25) (layer "B.Cu") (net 9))
 (segment (start 177.9 108.7) (end 179.505 107.095) (width 0.25) (layer "F.Cu") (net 4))
 (segment (start 179.57 72.55) (end 179.57 77.73) (width 0.25) (layer "F.Cu") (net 4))
 (segment (start 151.19 108.7) (end 177.9 108.7) (width 0.25) (layer "F.Cu") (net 4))
 (segment (start 147.87 105.38) (end 151.19 108.7) (width 0.25) (layer "F.Cu") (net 4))
 (segment (start 179.57 77.73) (end 179.4 77.9) (width 0.25) (layer "F.Cu") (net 4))
 (segment (start 177.9 108.8) (end 177.9 108.7) (width 0.25) (layer "F.Cu") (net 4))
 (via (at 175.9 110.8) (size 0.8) (drill 0.4) (layers "F.Cu" "B.Cu") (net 4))
 (via (at 179.4 77.9) (size 0.8) (drill 0.4) (layers "F.Cu" "B.Cu") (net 4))
 (segment (start 178.3 82.119589) (end 179.480411 83.3) (width 0.25) (layer "B.Cu") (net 4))
 (segment (start 179.480411 83.3) (end 179.5 83.3) (width 0.25) (layer "B.Cu") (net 4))
 (segment (start 179.47 123.8) (end 179.47 114.37) (width 0.25) (layer "B.Cu") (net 4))
 (segment (start 180.970489 105.629511) (end 180.970489 104.529511) (width 0.25) (layer "B.Cu") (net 4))
 (segment (start 179.505 107.095) (end 180.970489 105.629511) (width 0.25) (layer "B.Cu") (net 4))
 (segment (start 179.505 107.095) (end 177.205 107.095) (width 0.25) (layer "B.Cu") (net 4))
 (segment (start 177.205 107.095) (end 175.9 108.4) (width 0.25) (layer "B.Cu") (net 4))
 (segment (start 179.47 114.37) (end 175.9 110.8) (width 0.25) (layer "B.Cu") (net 4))
 (segment (start 185.7 103.7) (end 184.870489 104.529511) (width 0.25) (layer "B.Cu") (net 4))
 (segment (start 181.910411 87) (end 182.5 87) (width 0.25) (layer "B.Cu") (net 4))
 (segment (start 179.5 83.3) (end 179.505 83.305) (width 0.25) (layer "B.Cu") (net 4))
 (segment (start 179.505 84.345) (end 179.505 84.594589) (width 0.25) (layer "B.Cu") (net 4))
 (segment (start 179.505 84.594589) (end 181.910411 87) (width 0.25) (layer "B.Cu") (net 4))
 (segment (start 178.3 79) (end 178.3 82.119589) (width 0.25) (layer "B.Cu") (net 4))
 (segment (start 175.9 108.4) (end 175.9 110.8) (width 0.25) (layer "B.Cu") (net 4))
 (segment (start 179.505 83.305) (end 179.505 84.345) (width 0.25) (layer "B.Cu") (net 4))
 (segment (start 185.7 90.2) (end 185.7 103.7) (width 0.25) (layer "B.Cu") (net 4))
 (segment (start 184.870489 104.529511) (end 180.970489 104.529511) (width 0.25) (layer "B.Cu") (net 4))
 (segment (start 179.4 77.9) (end 178.3 79) (width 0.25) (layer "B.Cu") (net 4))
 (segment (start 182.5 87) (end 185.7 90.2) (width 0.25) (layer "B.Cu") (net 4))
 (segment (start 177.5 78.3) (end 177.824511 78.624511) (width 0.25) (layer "F.Cu") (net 3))
 (segment (start 181 80.640978) (end 180.970489 80.670489) (width 0.25) (layer "F.Cu") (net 3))
 (segment (start 152.83 107.8) (end 174.2 107.8) (width 0.25) (layer "F.Cu") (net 3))
 (segment (start 183.4 119.3) (end 181.43 119.3) (width 0.25) (layer "F.Cu") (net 3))
 (segment (start 179.924511 78.624511) (end 181 79.7) (width 0.25) (layer "F.Cu") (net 3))
 (segment (start 180.970489 80.670489) (end 180.970489 84.540489) (width 0.25) (layer "F.Cu") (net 3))
 (segment (start 177.824511 78.624511) (end 179.924511 78.624511) (width 0.25) (layer "F.Cu") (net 3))
 (segment (start 181 79.7) (end 181 80.640978) (width 0.25) (layer "F.Cu") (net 3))
 (segment (start 180.970489 84.540489) (end 182.045 85.615) (width 0.25) (layer "F.Cu") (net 3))
 (segment (start 181.43 119.3) (end 176.93 123.8) (width 0.25) (layer "F.Cu") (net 3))
 (segment (start 150.41 105.38) (end 152.83 107.8) (width 0.25) (layer "F.Cu") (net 3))
 (via (at 174.2 107.8) (size 0.8) (drill 0.4) (layers "F.Cu" "B.Cu") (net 3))
 (via (at 183.4 119.3) (size 0.8) (drill 0.4) (layers "F.Cu" "B.Cu") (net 3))
 (via (at 177.5 78.3) (size 0.8) (drill 0.4) (layers "F.Cu" "B.Cu") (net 3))
 (segment (start 183.4 109.72) (end 183.4 119.3) (width 0.25) (layer "B.Cu") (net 3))
 (segment (start 177.03 72.55) (end 177.03 77.83) (width 0.25) (layer "B.Cu") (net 3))
 (segment (start 182.045 85.615) (end 186.395479 89.965479) (width 0.25) (layer "B.Cu") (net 3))
 (segment (start 176.93 113.93) (end 174.2 111.2) (width 0.25) (layer "B.Cu") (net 3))
 (segment (start 176.93 123.8) (end 176.93 113.93) (width 0.25) (layer "B.Cu") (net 3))
 (segment (start 182.045 108.365) (end 183.4 109.72) (width 0.25) (layer "B.Cu") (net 3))
 (segment (start 186.395479 104.014521) (end 182.045 108.365) (width 0.25) (layer "B.Cu") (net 3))
 (segment (start 174.2 111.2) (end 174.2 107.8) (width 0.25) (layer "B.Cu") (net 3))
 (segment (start 186.395479 89.965479) (end 186.395479 104.014521) (width 0.25) (layer "B.Cu") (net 3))
 (segment (start 177.03 77.83) (end 177.5 78.3) (width 0.25) (layer "B.Cu") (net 3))
 (segment (start 160.68 110.98) (end 160.7 111) (width 0.25) (layer "F.Cu") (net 7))
 (segment (start 153.105 124.05) (end 155.3 121.855) (width 0.25) (layer "F.Cu") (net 7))
 (segment (start 158.03 105.38) (end 158.03 105.6055) (width 0.25) (layer "F.Cu") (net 7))
 (segment (start 158.03 105.6055) (end 159.5 107.0755) (width 0.25) (layer "F.Cu") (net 7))
 (segment (start 127.905 111.595) (end 128 111.5) (width 0.25) (layer "F.Cu") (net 7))
 (segment (start 158.315 110.98) (end 160.68 110.98) (width 0.25) (layer "F.Cu") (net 7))
 (segment (start 125.35 111.595) (end 127.905 111.595) (width 0.25) (layer "F.Cu") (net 7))
 (segment (start 158.03 110.695) (end 158.315 110.98) (width 0.25) (layer "F.Cu") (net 7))
 (segment (start 155.3 121.855) (end 155.3 118.5) (width 0.25) (layer "F.Cu") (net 7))
 (via (at 128 111.5) (size 0.8) (drill 0.4) (layers "F.Cu" "B.Cu") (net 7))
 (via (at 155.3 118.5) (size 0.8) (drill 0.4) (layers "F.Cu" "B.Cu") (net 7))
 (via (at 159.5 107.0755) (size 0.8) (drill 0.4) (layers "F.Cu" "B.Cu") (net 7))
 (via (at 160.7 111) (size 0.8) (drill 0.4) (layers "F.Cu" "B.Cu") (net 7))
 (segment (start 160.7 108.2755) (end 159.5 107.0755) (width 0.25) (layer "B.Cu") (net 7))
 (segment (start 128 111.5) (end 153.5 111.5) (width 0.25) (layer "B.Cu") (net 7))
 (segment (start 153.5 111.5) (end 155 113) (width 0.25) (layer "B.Cu") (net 7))
 (segment (start 155.1 113.1) (end 155.3 113.3) (width 0.25) (layer "B.Cu") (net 7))
 (segment (start 160.7 111) (end 160.7 108.2755) (width 0.25) (layer "B.Cu") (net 7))
 (segment (start 155 113) (end 155.1 113.1) (width 0.25) (layer "B.Cu") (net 7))
 (segment (start 159.5 107.0755) (end 159.5 108.5) (width 0.25) (layer "B.Cu") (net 7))
 (segment (start 159.5 108.5) (end 155 113) (width 0.25) (layer "B.Cu") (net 7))
 (segment (start 155.3 113.3) (end 155.3 118.5) (width 0.25) (layer "B.Cu") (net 7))
 (segment (start 174.34 114.8) (end 174.3 114.8) (width 1) (layer "F.Cu") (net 2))
 (segment (start 179.505 109.635) (end 176.14 113) (width 1) (layer "F.Cu") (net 2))
 (segment (start 179.505 86.885) (end 180.775 86.885) (width 1) (layer "F.Cu") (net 2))
 (segment (start 162.885 110.98) (end 163.78 110.98) (width 0.25) (layer "F.Cu") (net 2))
 (segment (start 166.65 113) (end 168.9 113) (width 0.25) (layer "F.Cu") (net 2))
 (segment (start 176.14 113) (end 174.34 114.8) (width 1) (layer "F.Cu") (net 2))
 (segment (start 184.6 102.5) (end 184.6 108.35) (width 1) (layer "F.Cu") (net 2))
 (segment (start 174.49 72.55) (end 174.49 81.87) (width 1) (layer "F.Cu") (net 2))
 (segment (start 184.6 108.35) (end 182.045 110.905) (width 1) (layer "F.Cu") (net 2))
 (segment (start 174.49 81.87) (end 179.505 86.885) (width 1) (layer "F.Cu") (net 2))
 (segment (start 176.14 113) (end 166.65 113) (width 1) (layer "F.Cu") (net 2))
 (segment (start 165.8 113) (end 166.65 113) (width 0.25) (layer "F.Cu") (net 2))
 (segment (start 163.78 110.98) (end 165.8 113) (width 0.25) (layer "F.Cu") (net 2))
 (segment (start 180.775 86.885) (end 182.045 88.155) (width 1) (layer "F.Cu") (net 2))
 (via (at 174.3 114.8) (size 0.8) (drill 0.4) (layers "F.Cu" "B.Cu") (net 2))
 (via (at 184.6 102.5) (size 0.8) (drill 0.4) (layers "F.Cu" "B.Cu") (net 2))
 (segment (start 135.31 74.69) (end 135.31 74.75) (width 1) (layer "B.Cu") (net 2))
 (segment (start 184.6 90.71) (end 184.6 102.5) (width 1) (layer "B.Cu") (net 2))
 (segment (start 182.045 88.155) (end 184.6 90.71) (width 1) (layer "B.Cu") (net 2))
 (segment (start 139 71) (end 135.31 74.69) (width 1) (layer "B.Cu") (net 2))
 (segment (start 174.3 123.71) (end 174.39 123.8) (width 1) (layer "B.Cu") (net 2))
 (segment (start 173.499022 71) (end 139 71) (width 1) (layer "B.Cu") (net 2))
 (segment (start 182.045 110.905) (end 180.775 110.905) (width 1) (layer "B.Cu") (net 2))
 (segment (start 180.775 110.905) (end 179.505 109.635) (width 1) (layer "B.Cu") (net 2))
 (segment (start 174.3 114.8) (end 174.3 123.71) (width 1) (layer "B.Cu") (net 2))
 (segment (start 174.49 71.990978) (end 173.499022 71) (width 1) (layer "B.Cu") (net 2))
 (segment (start 174.49 72.55) (end 174.49 71.990978) (width 1) (layer "B.Cu") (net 2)))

